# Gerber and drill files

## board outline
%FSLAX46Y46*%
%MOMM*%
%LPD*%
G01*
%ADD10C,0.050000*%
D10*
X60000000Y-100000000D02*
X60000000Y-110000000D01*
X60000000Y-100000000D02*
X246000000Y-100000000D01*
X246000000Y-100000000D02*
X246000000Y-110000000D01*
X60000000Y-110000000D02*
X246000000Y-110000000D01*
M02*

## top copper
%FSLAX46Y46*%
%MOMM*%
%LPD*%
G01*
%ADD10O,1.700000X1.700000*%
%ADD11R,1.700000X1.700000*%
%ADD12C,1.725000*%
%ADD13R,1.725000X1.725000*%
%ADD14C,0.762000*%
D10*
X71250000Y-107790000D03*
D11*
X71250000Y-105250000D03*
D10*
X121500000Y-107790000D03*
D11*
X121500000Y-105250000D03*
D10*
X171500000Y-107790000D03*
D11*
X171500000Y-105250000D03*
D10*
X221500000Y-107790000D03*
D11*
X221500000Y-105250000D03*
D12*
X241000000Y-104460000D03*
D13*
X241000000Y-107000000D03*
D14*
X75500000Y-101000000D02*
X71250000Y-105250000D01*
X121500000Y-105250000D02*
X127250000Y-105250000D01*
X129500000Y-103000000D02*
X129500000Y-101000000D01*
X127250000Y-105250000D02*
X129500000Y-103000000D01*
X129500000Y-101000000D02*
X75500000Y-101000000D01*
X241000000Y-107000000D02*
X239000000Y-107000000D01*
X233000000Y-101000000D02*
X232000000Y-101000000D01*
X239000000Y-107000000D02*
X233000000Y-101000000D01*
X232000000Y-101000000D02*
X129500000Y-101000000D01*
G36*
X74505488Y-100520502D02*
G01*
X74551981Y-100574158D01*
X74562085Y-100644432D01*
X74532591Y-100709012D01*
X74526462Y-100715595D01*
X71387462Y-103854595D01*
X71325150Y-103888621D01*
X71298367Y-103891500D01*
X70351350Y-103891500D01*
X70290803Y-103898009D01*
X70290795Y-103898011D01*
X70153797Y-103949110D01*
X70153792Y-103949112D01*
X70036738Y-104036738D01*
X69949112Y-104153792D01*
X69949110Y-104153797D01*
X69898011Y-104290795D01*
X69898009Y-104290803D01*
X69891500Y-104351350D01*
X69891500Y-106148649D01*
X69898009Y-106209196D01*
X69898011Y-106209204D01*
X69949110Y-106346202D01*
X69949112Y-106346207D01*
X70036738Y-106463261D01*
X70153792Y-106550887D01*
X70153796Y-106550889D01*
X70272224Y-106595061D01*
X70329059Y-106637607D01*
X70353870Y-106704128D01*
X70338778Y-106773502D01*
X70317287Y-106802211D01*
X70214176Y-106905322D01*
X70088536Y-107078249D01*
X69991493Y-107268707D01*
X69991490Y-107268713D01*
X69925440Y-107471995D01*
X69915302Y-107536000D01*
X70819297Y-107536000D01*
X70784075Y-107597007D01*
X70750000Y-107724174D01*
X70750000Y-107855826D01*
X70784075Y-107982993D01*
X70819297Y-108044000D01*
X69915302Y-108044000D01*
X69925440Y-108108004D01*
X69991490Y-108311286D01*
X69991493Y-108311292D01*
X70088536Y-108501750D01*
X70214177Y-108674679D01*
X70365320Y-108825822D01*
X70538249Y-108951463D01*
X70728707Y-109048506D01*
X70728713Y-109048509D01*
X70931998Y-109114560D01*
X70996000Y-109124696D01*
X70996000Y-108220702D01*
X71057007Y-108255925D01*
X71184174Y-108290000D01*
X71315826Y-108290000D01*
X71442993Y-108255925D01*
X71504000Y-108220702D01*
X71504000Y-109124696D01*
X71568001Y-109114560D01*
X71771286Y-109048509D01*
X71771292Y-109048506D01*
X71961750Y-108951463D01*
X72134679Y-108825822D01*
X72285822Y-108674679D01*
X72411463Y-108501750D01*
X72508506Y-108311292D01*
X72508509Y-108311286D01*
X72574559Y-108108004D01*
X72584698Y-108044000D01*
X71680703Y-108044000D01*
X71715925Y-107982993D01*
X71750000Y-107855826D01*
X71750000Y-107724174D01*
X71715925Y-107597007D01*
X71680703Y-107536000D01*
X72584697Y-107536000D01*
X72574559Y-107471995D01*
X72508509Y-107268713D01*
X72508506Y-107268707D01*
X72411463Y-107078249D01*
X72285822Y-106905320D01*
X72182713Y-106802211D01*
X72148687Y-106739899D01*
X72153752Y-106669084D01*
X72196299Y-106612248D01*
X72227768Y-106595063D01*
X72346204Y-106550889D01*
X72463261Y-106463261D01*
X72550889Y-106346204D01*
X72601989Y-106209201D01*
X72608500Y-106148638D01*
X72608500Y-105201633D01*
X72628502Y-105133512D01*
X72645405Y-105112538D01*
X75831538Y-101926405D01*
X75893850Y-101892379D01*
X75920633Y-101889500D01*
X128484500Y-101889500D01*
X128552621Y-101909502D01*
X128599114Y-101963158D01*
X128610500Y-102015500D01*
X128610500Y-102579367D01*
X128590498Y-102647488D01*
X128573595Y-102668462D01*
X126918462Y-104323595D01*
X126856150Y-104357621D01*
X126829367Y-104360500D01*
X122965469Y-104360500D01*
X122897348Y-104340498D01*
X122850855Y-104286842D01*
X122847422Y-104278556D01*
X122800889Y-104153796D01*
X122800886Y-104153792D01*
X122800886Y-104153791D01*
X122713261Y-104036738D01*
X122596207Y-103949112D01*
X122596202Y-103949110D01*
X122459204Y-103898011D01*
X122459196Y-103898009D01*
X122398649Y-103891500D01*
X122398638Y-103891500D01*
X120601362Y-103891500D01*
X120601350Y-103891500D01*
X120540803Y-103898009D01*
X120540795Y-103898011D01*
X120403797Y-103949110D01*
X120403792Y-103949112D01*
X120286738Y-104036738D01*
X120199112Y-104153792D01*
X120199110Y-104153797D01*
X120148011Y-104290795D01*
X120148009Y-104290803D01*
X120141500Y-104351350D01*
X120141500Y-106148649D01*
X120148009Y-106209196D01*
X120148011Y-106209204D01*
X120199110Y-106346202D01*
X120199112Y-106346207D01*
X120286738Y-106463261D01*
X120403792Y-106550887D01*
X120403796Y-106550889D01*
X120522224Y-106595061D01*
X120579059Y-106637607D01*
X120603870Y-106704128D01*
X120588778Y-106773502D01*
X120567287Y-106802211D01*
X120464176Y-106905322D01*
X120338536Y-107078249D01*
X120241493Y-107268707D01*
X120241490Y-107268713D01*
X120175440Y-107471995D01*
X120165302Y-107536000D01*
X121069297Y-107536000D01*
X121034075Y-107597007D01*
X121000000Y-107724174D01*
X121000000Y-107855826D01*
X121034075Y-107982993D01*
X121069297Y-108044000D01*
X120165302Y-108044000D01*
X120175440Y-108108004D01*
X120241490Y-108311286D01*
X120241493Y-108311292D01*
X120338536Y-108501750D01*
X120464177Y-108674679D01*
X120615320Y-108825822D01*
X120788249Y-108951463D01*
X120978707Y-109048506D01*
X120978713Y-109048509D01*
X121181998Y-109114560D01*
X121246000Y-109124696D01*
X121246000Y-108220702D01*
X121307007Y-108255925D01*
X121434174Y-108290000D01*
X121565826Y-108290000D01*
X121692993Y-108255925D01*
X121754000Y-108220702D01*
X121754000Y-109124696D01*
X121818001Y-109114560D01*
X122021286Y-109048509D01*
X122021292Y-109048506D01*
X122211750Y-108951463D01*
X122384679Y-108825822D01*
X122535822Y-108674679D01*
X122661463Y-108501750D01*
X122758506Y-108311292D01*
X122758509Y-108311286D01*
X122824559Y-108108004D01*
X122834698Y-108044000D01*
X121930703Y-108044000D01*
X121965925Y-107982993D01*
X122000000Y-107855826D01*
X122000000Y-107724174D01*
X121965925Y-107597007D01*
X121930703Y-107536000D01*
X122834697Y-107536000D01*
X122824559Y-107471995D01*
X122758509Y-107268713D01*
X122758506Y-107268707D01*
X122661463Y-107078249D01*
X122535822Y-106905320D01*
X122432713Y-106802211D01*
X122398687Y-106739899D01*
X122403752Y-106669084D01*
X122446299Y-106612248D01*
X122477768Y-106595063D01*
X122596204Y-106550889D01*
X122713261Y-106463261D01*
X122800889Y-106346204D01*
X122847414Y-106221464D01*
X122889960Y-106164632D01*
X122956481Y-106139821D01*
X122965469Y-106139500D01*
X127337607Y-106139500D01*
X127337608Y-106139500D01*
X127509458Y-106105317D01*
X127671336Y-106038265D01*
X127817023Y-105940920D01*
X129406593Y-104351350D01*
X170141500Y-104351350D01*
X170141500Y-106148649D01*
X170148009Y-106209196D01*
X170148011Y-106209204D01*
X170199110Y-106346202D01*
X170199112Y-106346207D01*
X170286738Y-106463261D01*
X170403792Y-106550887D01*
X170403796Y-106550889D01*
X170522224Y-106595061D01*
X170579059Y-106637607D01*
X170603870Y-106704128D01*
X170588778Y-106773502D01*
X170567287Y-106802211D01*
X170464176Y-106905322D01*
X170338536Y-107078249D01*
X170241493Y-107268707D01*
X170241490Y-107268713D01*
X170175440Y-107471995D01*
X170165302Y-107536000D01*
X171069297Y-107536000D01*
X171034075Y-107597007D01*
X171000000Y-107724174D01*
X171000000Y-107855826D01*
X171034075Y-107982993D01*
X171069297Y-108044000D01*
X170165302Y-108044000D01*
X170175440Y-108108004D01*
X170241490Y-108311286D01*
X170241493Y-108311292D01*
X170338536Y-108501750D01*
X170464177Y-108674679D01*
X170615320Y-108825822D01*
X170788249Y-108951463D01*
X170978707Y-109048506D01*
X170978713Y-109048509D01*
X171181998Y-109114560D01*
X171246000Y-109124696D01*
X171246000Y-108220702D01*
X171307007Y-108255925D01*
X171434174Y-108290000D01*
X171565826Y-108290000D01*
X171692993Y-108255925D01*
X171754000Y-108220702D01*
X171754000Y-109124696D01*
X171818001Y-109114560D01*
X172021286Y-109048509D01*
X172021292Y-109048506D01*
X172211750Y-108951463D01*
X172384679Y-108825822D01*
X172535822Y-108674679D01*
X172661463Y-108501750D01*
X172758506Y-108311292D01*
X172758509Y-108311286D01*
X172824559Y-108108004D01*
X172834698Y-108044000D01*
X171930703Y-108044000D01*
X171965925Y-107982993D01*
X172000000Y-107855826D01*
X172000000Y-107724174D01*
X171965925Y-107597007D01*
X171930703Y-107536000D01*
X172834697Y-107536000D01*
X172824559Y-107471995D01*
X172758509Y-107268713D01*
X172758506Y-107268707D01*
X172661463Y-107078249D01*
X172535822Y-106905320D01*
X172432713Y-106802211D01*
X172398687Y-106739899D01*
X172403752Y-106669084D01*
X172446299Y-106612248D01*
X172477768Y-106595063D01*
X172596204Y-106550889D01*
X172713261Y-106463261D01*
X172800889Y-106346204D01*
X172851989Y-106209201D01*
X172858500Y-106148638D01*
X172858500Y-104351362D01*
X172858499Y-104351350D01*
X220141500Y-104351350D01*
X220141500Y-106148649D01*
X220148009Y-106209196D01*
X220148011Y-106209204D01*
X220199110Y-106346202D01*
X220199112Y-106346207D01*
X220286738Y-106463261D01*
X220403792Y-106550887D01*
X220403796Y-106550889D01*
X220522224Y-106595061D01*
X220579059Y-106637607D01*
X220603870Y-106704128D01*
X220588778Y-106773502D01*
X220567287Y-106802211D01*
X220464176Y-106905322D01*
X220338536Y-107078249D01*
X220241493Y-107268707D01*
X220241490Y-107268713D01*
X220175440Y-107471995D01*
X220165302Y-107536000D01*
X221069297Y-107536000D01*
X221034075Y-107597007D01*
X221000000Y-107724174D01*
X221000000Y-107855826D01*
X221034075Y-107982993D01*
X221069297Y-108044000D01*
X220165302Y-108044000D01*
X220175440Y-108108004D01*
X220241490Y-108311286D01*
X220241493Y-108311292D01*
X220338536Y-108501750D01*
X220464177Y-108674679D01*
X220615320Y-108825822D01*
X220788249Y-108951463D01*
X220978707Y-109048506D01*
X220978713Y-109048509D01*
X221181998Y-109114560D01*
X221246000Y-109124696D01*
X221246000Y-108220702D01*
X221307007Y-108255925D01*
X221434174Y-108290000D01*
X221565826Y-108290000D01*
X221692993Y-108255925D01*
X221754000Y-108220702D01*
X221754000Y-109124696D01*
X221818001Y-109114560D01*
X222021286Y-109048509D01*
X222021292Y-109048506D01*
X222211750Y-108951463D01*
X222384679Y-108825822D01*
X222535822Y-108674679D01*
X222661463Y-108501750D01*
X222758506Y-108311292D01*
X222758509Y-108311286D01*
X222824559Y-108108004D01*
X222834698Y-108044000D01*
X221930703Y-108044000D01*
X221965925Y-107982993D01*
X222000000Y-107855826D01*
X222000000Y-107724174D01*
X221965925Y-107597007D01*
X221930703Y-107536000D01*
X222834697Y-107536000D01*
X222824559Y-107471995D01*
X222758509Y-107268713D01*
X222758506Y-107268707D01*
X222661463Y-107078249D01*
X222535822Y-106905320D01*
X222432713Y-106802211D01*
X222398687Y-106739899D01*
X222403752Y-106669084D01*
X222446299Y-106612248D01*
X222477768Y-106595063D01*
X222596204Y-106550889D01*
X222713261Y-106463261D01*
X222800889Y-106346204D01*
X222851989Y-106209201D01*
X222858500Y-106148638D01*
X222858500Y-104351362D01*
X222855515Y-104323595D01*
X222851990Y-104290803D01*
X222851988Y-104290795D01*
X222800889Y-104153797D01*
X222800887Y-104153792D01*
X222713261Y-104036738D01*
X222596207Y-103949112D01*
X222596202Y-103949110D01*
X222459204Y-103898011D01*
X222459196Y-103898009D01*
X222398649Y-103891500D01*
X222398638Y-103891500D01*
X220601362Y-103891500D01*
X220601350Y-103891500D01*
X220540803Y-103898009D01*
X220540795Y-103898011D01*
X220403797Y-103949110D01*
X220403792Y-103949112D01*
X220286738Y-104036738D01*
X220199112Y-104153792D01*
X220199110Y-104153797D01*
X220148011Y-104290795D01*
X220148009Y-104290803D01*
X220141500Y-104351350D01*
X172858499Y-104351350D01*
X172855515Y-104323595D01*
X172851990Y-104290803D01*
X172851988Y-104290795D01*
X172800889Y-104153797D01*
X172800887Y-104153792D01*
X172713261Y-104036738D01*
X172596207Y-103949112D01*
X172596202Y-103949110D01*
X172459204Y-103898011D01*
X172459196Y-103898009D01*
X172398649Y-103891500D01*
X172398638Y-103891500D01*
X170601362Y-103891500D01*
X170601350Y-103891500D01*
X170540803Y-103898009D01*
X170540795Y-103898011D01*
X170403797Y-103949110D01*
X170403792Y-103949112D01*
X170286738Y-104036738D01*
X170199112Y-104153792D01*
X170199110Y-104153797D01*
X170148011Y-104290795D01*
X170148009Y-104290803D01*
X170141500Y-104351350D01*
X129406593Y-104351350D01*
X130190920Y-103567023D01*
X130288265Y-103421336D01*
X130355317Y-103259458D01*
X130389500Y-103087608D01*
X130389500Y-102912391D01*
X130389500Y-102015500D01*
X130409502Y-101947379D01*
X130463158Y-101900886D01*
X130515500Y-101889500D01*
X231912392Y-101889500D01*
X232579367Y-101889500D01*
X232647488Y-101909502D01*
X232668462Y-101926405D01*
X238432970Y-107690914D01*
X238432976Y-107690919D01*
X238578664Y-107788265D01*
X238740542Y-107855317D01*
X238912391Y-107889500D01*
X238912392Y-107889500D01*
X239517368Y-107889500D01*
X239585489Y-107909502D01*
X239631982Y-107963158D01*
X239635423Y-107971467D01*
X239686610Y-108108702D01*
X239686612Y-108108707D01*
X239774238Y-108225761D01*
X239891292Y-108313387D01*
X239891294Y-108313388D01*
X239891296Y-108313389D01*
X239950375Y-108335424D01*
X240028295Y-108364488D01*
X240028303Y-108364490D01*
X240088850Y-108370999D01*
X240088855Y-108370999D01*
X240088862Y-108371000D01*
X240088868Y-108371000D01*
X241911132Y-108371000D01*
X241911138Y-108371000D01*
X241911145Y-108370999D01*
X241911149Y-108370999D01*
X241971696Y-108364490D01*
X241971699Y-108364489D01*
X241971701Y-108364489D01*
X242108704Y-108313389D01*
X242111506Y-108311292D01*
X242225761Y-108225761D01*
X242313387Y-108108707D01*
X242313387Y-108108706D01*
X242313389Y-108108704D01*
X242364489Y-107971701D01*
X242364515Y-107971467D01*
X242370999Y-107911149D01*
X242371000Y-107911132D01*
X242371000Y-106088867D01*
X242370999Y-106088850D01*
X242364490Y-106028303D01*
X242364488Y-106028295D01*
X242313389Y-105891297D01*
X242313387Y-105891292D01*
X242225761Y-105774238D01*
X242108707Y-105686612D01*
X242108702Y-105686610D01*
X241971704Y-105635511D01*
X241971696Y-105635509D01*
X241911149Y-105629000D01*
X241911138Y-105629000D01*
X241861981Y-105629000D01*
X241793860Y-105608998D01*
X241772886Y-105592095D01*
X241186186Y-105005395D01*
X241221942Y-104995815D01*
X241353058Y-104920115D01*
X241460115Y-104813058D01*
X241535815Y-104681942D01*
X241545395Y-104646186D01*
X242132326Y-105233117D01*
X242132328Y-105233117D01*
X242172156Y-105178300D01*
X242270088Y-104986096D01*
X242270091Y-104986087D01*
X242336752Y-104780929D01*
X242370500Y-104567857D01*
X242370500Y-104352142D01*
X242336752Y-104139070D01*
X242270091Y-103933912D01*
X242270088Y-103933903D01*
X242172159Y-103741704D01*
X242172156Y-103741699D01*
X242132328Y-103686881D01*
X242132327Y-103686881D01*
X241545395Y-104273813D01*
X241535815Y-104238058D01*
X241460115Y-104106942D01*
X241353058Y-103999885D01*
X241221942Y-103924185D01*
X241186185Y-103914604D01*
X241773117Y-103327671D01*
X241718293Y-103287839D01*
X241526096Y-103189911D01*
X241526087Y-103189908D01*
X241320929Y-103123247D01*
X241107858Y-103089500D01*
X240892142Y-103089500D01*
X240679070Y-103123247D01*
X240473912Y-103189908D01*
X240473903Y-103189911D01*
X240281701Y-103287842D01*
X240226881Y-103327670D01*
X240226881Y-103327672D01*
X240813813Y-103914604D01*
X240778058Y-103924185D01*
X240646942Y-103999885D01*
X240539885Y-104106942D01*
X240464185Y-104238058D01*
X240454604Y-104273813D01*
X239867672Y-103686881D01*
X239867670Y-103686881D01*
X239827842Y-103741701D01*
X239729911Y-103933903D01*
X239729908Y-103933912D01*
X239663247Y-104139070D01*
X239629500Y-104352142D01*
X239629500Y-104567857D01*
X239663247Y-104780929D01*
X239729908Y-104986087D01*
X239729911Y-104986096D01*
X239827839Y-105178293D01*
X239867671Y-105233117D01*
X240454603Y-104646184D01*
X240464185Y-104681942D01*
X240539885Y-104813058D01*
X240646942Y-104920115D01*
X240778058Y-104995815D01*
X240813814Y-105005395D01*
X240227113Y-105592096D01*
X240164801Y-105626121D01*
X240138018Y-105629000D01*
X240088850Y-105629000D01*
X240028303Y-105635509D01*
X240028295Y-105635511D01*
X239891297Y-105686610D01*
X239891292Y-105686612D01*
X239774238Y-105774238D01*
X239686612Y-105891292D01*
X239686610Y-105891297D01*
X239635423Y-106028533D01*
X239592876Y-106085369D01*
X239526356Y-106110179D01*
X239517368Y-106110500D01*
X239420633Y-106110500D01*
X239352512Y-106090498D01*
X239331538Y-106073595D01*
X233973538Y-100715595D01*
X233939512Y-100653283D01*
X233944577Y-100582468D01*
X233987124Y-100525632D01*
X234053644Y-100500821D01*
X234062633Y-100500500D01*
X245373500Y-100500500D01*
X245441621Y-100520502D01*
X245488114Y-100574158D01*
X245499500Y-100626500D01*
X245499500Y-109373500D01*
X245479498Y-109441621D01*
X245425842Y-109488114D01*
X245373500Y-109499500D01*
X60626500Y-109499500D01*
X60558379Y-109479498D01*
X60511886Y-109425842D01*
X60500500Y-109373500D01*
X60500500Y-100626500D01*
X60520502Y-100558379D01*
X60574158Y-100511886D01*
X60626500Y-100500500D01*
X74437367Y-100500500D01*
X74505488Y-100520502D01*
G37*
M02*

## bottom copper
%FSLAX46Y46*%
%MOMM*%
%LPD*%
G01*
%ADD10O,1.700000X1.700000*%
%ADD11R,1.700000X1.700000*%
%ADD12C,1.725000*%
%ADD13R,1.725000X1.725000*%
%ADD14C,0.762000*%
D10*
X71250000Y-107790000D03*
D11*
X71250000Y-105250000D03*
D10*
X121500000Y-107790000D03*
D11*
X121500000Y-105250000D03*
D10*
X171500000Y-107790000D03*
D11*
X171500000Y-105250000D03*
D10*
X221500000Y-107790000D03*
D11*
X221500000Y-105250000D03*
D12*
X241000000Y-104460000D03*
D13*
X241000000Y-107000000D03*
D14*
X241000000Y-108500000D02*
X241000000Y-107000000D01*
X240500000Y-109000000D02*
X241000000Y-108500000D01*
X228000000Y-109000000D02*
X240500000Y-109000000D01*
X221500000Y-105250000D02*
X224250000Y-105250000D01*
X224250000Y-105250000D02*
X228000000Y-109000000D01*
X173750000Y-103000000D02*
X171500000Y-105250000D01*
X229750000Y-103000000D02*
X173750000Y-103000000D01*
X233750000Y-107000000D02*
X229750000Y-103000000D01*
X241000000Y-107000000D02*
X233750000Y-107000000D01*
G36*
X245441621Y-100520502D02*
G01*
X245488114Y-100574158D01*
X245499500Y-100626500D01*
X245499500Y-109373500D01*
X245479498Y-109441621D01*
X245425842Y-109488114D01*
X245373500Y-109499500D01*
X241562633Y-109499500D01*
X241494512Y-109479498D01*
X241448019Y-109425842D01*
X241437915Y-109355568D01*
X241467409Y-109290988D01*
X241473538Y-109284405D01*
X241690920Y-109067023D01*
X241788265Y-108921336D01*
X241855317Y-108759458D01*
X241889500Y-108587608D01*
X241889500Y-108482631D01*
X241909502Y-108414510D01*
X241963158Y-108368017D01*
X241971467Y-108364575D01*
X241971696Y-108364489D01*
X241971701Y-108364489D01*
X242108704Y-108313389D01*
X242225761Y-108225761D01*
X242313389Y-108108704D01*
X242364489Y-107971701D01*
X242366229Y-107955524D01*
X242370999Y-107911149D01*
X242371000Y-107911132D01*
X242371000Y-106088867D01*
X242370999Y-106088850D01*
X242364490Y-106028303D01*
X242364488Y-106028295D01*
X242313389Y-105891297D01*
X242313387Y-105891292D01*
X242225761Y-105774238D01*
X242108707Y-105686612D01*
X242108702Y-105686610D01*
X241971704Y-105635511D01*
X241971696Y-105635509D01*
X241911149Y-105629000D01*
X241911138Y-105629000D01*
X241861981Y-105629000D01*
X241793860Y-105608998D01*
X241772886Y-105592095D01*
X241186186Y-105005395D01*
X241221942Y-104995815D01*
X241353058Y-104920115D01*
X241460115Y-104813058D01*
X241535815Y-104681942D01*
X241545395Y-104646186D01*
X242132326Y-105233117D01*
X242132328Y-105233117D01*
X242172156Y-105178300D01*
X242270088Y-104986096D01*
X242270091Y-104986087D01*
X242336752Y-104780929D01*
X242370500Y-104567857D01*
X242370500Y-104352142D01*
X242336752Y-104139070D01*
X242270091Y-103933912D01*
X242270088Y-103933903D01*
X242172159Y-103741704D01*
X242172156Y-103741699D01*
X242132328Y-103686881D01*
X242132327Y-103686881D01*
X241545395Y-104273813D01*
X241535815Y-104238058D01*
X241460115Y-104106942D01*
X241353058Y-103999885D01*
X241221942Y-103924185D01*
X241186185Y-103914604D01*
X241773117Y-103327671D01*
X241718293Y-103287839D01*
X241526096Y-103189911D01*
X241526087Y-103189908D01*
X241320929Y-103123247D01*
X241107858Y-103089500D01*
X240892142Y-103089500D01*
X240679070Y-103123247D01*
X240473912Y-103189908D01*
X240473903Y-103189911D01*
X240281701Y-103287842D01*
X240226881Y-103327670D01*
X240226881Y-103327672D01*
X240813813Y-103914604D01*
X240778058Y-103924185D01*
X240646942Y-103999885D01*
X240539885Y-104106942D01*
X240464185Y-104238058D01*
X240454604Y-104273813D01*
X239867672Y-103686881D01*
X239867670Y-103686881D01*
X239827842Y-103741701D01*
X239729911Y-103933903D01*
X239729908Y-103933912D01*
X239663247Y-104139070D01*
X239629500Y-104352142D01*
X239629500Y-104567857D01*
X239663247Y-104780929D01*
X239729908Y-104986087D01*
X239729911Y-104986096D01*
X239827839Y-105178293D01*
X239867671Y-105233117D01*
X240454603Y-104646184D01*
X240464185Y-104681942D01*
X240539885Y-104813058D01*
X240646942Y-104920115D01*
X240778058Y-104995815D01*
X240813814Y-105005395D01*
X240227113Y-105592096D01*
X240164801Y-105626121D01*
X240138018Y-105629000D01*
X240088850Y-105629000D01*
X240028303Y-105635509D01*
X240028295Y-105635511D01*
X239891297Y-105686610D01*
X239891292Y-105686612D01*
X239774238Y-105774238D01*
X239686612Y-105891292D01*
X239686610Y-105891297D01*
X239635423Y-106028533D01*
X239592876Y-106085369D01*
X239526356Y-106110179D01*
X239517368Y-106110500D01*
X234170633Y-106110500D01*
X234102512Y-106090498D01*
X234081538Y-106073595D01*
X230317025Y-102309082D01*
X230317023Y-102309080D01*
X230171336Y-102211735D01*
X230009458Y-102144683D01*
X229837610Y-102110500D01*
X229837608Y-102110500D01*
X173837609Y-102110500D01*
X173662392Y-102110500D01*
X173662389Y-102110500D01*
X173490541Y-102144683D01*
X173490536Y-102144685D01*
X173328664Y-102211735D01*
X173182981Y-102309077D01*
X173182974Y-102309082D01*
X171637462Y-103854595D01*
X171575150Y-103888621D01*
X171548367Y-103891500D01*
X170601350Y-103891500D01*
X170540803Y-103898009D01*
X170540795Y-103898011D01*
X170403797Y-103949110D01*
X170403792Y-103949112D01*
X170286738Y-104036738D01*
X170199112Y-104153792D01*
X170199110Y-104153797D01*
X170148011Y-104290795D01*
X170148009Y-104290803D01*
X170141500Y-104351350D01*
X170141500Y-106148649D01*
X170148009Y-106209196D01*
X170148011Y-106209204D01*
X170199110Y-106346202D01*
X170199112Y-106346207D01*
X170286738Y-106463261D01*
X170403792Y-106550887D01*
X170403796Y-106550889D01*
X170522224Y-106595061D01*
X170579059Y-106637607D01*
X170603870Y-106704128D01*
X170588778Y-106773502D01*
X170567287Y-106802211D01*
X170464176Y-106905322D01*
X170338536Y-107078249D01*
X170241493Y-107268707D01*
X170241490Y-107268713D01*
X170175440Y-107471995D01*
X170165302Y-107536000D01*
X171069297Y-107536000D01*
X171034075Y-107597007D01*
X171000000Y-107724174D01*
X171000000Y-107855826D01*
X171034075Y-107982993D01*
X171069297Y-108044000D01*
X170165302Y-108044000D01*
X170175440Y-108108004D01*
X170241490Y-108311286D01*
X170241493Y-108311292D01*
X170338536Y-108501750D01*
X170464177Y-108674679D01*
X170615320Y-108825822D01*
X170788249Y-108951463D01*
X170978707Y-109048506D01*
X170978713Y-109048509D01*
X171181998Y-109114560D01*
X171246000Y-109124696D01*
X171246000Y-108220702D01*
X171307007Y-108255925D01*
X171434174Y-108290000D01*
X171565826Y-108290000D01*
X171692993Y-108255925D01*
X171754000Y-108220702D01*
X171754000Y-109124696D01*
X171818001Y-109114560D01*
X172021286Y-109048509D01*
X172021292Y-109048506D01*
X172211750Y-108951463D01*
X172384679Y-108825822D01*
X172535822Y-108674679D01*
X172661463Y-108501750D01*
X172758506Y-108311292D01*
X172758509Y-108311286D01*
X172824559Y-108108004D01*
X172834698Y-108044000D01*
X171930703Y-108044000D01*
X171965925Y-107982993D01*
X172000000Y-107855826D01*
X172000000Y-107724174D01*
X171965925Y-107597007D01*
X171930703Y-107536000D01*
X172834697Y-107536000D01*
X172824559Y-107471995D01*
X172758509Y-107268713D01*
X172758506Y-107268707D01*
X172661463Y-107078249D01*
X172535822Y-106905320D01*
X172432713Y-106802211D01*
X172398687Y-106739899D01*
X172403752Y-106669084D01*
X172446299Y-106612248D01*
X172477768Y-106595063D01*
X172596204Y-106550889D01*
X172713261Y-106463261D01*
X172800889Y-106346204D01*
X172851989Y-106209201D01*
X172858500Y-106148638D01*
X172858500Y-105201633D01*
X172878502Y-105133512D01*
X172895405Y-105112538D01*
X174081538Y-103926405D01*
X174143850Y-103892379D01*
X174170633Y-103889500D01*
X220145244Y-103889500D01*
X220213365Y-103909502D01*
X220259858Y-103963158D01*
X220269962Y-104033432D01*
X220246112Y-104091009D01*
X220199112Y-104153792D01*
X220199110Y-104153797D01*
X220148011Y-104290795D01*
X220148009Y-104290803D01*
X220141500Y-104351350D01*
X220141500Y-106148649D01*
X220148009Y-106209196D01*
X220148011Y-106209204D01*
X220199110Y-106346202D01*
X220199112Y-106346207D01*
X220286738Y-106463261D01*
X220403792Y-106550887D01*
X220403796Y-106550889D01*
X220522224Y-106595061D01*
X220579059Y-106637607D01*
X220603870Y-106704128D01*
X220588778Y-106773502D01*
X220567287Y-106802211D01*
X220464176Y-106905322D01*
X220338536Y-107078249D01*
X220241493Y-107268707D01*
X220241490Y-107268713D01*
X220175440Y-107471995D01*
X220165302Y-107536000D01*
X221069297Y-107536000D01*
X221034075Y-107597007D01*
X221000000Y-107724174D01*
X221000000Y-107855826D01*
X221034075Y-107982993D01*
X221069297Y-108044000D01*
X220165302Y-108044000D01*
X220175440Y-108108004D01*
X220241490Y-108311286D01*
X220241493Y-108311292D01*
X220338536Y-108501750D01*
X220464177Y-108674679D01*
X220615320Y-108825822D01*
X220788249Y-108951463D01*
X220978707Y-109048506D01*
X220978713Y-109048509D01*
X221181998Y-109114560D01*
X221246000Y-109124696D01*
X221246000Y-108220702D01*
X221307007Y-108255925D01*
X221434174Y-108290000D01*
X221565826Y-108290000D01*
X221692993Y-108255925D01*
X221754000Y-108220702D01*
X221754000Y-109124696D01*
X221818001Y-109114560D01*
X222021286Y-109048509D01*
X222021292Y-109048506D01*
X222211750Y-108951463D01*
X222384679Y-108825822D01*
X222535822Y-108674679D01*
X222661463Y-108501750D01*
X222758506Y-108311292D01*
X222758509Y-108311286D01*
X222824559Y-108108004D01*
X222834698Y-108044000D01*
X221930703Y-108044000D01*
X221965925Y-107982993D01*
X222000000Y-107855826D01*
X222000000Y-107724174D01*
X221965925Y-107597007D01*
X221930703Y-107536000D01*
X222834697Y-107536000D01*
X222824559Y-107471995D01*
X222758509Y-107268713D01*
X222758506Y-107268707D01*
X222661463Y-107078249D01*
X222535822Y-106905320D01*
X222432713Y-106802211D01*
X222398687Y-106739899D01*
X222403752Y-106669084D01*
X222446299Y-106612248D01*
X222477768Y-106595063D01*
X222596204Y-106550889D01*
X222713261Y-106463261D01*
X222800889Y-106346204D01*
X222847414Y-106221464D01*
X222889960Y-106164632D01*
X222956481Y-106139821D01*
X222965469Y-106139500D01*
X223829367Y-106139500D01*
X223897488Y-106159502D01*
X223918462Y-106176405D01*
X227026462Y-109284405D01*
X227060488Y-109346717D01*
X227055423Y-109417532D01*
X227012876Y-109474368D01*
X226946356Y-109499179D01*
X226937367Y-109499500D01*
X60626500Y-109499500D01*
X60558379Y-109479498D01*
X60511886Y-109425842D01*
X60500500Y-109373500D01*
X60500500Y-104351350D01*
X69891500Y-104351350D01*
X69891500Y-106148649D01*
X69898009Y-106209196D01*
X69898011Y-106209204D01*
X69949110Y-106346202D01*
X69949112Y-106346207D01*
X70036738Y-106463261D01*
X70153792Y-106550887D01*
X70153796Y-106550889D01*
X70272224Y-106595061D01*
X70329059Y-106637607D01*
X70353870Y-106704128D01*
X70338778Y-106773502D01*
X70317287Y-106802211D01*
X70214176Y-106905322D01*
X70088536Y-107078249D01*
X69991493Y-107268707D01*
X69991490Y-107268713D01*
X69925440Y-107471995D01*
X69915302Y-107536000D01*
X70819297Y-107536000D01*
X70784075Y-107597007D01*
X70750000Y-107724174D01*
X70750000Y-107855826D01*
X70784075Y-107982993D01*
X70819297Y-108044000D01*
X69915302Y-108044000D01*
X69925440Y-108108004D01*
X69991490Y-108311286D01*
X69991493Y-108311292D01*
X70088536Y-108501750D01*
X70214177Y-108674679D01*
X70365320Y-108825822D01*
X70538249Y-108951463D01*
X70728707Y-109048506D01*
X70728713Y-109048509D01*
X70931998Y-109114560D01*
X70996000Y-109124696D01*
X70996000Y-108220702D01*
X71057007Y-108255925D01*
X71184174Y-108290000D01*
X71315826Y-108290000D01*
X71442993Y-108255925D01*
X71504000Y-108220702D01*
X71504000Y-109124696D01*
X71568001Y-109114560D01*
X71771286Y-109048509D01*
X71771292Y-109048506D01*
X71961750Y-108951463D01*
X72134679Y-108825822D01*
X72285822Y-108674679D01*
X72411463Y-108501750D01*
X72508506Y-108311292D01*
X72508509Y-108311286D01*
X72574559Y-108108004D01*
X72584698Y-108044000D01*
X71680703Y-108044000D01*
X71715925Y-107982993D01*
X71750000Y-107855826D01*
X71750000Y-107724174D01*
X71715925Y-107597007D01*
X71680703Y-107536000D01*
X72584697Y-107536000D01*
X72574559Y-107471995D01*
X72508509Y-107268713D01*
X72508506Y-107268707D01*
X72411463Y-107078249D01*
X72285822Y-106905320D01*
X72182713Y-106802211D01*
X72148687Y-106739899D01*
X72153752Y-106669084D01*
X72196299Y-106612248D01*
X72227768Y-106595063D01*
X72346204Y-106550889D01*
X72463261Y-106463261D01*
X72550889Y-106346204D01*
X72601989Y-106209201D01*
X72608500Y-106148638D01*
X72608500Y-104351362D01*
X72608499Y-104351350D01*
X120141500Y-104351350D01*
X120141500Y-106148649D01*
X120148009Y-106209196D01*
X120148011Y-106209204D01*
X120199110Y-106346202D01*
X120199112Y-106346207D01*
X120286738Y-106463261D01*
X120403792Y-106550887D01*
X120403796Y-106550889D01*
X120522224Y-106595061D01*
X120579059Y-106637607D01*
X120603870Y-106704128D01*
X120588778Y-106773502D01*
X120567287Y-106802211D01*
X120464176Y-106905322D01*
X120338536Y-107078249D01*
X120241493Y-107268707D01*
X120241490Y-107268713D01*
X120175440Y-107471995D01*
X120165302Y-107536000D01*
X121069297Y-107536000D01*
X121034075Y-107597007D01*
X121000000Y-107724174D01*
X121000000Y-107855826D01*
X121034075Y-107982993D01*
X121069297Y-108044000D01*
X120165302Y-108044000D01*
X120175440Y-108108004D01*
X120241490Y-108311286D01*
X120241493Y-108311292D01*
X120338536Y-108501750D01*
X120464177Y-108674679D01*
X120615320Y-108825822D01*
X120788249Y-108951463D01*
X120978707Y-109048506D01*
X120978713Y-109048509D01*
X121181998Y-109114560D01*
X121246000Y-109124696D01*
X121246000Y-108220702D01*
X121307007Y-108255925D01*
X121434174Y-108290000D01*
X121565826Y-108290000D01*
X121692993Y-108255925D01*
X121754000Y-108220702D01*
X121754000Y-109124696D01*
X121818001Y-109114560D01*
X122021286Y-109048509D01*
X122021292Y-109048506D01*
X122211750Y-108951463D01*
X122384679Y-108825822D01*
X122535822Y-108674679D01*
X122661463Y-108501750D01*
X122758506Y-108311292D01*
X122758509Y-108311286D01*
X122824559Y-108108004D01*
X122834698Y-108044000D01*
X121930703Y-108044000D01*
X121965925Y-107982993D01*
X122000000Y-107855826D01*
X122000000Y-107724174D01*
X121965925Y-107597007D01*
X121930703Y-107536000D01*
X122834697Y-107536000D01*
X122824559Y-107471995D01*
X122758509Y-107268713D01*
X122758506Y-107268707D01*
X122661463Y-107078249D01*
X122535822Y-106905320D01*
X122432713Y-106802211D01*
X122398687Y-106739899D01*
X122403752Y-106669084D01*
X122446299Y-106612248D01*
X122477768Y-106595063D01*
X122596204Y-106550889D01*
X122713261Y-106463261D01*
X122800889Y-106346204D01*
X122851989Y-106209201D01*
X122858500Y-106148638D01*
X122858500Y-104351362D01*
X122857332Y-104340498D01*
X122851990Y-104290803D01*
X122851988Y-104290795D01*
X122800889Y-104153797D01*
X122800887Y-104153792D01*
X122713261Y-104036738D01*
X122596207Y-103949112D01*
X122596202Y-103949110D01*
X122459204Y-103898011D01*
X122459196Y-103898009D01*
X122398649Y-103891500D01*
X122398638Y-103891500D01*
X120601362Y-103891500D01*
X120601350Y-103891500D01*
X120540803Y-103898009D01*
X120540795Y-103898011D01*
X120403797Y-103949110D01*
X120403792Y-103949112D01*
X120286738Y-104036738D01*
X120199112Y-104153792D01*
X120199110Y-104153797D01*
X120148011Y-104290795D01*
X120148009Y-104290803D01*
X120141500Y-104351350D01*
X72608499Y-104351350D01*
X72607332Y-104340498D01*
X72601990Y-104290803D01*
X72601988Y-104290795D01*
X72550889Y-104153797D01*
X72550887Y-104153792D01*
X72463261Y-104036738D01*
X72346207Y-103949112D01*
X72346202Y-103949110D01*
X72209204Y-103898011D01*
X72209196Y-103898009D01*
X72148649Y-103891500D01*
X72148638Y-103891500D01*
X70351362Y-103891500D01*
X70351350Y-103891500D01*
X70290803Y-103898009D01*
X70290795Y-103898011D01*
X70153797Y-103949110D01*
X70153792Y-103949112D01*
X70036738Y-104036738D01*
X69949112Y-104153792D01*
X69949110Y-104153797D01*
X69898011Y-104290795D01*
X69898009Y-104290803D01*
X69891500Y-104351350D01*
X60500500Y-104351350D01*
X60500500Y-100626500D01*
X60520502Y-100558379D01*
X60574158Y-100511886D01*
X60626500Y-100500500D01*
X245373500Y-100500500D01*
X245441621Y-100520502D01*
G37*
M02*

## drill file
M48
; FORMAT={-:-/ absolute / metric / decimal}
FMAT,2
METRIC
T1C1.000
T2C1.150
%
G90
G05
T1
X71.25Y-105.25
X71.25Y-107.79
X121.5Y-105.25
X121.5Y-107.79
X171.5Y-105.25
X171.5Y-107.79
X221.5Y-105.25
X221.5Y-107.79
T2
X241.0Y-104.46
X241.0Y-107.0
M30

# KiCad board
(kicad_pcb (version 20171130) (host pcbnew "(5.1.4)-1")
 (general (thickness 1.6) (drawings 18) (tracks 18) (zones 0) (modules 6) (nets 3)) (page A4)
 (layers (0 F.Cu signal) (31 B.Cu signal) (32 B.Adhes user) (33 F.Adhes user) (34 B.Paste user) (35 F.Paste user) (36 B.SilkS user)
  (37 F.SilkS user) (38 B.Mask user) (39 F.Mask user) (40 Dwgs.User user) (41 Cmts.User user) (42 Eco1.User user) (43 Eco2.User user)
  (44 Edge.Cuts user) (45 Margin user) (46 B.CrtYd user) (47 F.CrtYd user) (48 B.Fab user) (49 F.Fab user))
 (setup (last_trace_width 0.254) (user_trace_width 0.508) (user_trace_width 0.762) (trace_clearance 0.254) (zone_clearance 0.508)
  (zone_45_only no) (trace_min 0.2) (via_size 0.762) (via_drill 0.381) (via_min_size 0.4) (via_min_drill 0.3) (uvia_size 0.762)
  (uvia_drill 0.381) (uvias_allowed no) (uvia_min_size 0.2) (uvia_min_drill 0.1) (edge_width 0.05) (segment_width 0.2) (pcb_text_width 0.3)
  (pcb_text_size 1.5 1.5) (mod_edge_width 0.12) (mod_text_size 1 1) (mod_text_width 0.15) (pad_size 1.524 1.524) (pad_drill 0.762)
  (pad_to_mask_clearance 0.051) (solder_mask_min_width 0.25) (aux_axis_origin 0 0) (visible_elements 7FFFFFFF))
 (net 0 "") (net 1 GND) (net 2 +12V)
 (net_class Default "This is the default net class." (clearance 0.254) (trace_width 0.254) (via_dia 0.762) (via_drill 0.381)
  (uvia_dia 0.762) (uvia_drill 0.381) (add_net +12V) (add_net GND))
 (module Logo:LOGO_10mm (layer F.Cu) (at 149 105.25)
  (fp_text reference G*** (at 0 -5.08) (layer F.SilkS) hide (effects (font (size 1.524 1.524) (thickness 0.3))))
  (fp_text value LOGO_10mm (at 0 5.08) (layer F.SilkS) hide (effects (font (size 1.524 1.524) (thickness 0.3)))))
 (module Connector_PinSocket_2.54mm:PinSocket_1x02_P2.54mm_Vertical (layer F.Cu) (at 71.25 105.25)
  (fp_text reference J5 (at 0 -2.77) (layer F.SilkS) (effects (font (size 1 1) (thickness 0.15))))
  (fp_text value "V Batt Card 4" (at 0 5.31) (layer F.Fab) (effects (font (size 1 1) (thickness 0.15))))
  (pad 2 thru_hole oval (at 0 2.54) (size 1.7 1.7) (drill 1) (layers *.Cu *.Mask) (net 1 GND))
  (pad 1 thru_hole rect (at 0 0) (size 1.7 1.7) (drill 1) (layers *.Cu *.Mask) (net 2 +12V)))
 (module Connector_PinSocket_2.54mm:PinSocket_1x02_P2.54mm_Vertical (layer F.Cu) (at 121.5 105.25)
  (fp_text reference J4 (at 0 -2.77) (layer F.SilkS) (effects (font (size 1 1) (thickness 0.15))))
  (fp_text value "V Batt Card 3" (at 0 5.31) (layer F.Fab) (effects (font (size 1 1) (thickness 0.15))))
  (pad 2 thru_hole oval (at 0 2.54) (size 1.7 1.7) (drill 1) (layers *.Cu *.Mask) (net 1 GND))
  (pad 1 thru_hole rect (at 0 0) (size 1.7 1.7) (drill 1) (layers *.Cu *.Mask) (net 2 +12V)))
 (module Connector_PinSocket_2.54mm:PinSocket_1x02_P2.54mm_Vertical (layer F.Cu) (at 171.5 105.25)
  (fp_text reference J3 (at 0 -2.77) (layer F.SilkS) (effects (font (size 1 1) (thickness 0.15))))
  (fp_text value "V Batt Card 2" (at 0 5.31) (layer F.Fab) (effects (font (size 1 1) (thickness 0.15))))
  (pad 2 thru_hole oval (at 0 2.54) (size 1.7 1.7) (drill 1) (layers *.Cu *.Mask) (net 1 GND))
  (pad 1 thru_hole rect (at 0 0) (size 1.7 1.7) (drill 1) (layers *.Cu *.Mask) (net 2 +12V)))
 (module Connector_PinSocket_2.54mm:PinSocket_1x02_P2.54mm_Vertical (layer F.Cu) (at 221.5 105.25)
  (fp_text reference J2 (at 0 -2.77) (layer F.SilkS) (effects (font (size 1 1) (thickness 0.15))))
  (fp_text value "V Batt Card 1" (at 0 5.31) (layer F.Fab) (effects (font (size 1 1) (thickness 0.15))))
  (pad 2 thru_hole oval (at 0 2.54) (size 1.7 1.7) (drill 1) (layers *.Cu *.Mask) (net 1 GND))
  (pad 1 thru_hole rect (at 0 0) (size 1.7 1.7) (drill 1) (layers *.Cu *.Mask) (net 2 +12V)))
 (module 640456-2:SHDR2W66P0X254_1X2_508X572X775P (layer F.Cu) (at 241 107 90)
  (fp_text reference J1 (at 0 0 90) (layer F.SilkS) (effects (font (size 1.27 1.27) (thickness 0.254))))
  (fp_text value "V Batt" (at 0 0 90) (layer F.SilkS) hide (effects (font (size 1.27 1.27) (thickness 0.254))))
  (pad 2 thru_hole circle (at 2.54 0 180) (size 1.725 1.725) (drill 1.15) (layers *.Cu *.Mask F.SilkS) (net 1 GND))
  (pad 1 thru_hole rect (at 0 0 180) (size 1.725 1.725) (drill 1.15) (layers *.Cu *.Mask F.SilkS) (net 2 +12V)))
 (gr_line (start 60 100) (end 60 110) (layer Edge.Cuts) (width 0.05))
 (gr_line (start 60 100) (end 246 100) (layer Edge.Cuts) (width 0.05))
 (gr_line (start 246 100) (end 246 110) (layer Edge.Cuts) (width 0.05))
 (gr_line (start 60 110) (end 246 110) (layer Edge.Cuts) (width 0.05))
 (segment (start 75.5 101) (end 71.25 105.25) (width 0.762) (layer F.Cu) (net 2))
 (segment (start 121.5 105.25) (end 127.25 105.25) (width 0.762) (layer F.Cu) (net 2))
 (segment (start 129.5 103) (end 129.5 101) (width 0.762) (layer F.Cu) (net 2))
 (segment (start 127.25 105.25) (end 129.5 103) (width 0.762) (layer F.Cu) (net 2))
 (segment (start 129.5 101) (end 75.5 101) (width 0.762) (layer F.Cu) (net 2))
 (segment (start 241 108.5) (end 241 107) (width 0.762) (layer B.Cu) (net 2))
 (segment (start 240.5 109) (end 241 108.5) (width 0.762) (layer B.Cu) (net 2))
 (segment (start 228 109) (end 240.5 109) (width 0.762) (layer B.Cu) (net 2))
 (segment (start 221.5 105.25) (end 224.25 105.25) (width 0.762) (layer B.Cu) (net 2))
 (segment (start 224.25 105.25) (end 228 109) (width 0.762) (layer B.Cu) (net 2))
 (segment (start 173.75 103) (end 171.5 105.25) (width 0.762) (layer B.Cu) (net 2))
 (segment (start 229.75 103) (end 173.75 103) (width 0.762) (layer B.Cu) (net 2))
 (segment (start 233.75 107) (end 229.75 103) (width 0.762) (layer B.Cu) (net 2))
 (segment (start 241 107) (end 233.75 107) (width 0.762) (layer B.Cu) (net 2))
 (segment (start 241 107) (end 239 107) (width 0.762) (layer F.Cu) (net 2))
 (segment (start 233 101) (end 232 101) (width 0.762) (layer F.Cu) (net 2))
 (segment (start 239 107) (end 233 101) (width 0.762) (layer F.Cu) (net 2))
 (segment (start 232 101) (end 129.5 101) (width 0.762) (layer F.Cu) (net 2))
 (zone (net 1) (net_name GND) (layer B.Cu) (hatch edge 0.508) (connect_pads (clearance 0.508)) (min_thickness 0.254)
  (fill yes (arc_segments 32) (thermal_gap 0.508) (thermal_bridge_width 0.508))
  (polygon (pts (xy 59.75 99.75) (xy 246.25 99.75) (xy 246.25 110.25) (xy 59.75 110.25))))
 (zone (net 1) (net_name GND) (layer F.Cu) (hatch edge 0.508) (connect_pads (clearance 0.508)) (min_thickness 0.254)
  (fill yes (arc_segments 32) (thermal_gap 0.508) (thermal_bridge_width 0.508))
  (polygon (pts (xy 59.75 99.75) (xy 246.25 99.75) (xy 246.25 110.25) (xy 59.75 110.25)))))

